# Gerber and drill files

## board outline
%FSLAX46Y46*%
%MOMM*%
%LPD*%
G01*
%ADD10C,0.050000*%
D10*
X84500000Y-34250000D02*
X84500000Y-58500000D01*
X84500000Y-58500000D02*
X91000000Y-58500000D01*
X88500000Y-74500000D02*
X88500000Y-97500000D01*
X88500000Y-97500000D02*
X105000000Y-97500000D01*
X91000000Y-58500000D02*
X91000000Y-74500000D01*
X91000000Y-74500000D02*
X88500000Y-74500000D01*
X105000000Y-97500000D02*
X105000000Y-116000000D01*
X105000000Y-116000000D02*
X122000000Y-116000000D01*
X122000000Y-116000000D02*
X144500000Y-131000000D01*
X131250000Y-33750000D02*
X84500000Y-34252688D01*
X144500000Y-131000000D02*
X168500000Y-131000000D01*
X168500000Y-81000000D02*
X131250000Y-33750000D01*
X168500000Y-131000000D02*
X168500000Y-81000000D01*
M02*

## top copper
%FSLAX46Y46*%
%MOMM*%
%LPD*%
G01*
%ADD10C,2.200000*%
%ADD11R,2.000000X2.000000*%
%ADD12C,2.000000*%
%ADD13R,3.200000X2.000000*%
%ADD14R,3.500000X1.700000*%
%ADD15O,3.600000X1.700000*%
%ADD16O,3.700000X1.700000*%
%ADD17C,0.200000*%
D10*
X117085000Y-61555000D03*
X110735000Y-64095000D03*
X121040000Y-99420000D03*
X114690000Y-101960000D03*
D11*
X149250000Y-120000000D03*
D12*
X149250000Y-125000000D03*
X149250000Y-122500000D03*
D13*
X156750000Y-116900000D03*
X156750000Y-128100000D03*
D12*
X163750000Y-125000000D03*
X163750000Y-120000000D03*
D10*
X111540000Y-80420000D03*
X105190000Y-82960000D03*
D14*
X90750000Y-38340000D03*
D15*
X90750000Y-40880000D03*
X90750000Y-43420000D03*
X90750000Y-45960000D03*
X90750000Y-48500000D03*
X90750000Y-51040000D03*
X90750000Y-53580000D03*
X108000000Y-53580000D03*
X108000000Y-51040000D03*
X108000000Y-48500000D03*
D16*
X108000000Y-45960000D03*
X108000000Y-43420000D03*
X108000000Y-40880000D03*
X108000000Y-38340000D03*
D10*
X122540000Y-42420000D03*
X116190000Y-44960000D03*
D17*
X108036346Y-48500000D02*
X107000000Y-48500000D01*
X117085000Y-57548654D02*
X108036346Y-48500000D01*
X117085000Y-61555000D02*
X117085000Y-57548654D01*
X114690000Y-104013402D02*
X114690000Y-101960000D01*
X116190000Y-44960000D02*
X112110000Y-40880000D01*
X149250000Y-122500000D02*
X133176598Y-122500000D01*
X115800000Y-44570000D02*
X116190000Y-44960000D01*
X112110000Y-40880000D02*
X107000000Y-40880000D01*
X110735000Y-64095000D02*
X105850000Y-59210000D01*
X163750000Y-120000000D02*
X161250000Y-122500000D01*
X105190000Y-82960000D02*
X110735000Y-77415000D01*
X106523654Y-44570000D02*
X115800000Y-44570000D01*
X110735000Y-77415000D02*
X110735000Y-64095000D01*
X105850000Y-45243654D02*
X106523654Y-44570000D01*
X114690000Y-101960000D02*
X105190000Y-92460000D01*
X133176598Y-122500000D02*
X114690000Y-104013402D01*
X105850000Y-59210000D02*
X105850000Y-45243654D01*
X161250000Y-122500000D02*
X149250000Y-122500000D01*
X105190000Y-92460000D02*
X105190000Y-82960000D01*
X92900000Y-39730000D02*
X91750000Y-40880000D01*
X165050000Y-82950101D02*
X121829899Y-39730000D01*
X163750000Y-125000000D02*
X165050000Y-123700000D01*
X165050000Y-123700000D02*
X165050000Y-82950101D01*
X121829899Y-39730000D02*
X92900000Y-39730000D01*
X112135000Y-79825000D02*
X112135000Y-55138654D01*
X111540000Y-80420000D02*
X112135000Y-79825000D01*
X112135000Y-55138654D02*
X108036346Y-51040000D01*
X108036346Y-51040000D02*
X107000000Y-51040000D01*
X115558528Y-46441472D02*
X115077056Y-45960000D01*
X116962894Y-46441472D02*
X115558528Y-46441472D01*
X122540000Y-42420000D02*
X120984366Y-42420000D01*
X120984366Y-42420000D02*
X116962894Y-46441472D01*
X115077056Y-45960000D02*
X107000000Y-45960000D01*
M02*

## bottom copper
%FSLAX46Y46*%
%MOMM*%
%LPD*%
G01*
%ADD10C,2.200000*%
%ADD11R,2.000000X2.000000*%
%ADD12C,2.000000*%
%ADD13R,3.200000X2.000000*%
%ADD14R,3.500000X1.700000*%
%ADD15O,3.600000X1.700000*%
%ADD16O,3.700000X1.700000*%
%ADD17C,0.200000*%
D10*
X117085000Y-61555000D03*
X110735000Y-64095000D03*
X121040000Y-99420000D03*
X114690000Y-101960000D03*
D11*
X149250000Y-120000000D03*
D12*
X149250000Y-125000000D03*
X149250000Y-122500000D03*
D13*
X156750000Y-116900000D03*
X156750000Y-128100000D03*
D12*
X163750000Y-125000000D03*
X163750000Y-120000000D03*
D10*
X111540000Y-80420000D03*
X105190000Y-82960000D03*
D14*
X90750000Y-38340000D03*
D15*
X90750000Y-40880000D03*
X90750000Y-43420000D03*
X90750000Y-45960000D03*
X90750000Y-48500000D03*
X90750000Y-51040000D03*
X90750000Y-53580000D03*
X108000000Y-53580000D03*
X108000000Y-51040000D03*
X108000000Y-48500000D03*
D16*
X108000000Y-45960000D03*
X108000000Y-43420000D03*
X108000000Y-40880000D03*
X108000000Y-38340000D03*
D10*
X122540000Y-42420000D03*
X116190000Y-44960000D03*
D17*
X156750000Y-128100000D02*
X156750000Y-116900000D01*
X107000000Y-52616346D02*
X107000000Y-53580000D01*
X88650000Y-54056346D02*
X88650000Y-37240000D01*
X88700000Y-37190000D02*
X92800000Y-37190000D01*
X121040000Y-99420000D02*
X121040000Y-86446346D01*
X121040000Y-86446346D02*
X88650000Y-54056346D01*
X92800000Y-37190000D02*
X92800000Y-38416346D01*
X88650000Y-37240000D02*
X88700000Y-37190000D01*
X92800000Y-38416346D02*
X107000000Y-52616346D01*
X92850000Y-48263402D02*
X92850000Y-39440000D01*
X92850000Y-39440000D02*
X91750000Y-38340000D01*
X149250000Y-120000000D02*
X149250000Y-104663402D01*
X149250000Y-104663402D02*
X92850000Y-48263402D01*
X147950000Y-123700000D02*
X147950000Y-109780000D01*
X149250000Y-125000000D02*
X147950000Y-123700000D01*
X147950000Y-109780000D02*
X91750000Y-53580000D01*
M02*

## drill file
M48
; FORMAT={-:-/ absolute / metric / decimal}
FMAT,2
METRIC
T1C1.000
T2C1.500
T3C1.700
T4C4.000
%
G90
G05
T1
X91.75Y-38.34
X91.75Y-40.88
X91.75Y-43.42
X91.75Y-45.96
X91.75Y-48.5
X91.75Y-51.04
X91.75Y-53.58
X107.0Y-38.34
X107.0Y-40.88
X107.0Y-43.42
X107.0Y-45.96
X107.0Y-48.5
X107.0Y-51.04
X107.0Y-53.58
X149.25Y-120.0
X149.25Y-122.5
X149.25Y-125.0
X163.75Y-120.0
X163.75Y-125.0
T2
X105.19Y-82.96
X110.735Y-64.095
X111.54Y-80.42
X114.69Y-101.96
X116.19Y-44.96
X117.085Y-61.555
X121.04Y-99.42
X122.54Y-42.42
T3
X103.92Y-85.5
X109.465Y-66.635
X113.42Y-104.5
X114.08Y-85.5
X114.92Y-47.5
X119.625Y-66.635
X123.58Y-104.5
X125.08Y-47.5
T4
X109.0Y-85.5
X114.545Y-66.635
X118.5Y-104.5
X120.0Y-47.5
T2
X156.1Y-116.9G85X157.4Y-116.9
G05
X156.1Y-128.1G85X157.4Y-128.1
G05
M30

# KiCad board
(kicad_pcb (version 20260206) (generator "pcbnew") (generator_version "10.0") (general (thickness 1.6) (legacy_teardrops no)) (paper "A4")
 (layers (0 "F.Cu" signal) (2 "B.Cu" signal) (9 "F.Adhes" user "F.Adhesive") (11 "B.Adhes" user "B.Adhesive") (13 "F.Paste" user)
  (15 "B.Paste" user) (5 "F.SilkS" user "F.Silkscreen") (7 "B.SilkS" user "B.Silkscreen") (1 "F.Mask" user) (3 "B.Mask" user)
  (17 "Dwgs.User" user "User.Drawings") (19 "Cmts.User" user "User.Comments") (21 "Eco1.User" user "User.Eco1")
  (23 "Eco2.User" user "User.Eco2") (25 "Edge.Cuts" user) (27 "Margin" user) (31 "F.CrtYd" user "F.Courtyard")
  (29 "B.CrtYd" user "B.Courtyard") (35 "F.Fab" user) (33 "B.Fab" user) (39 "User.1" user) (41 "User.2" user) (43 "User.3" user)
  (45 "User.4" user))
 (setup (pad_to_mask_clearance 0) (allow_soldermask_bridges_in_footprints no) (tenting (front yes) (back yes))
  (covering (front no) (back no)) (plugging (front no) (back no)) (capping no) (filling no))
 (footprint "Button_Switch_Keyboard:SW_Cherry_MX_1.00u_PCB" (layer "F.Cu") (at 117.085 61.555)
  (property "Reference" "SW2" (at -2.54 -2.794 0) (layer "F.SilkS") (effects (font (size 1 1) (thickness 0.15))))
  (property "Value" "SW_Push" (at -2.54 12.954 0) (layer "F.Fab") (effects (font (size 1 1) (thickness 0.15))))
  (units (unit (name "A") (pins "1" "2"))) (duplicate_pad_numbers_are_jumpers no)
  (pad "" np_thru_hole circle (at -7.62 5.08) (size 1.7 1.7) (drill 1.7) (layers "*.Cu" "*.Mask"))
  (pad "" np_thru_hole circle (at -2.54 5.08) (size 4 4) (drill 4) (layers "*.Cu" "*.Mask"))
  (pad "" np_thru_hole circle (at 2.54 5.08) (size 1.7 1.7) (drill 1.7) (layers "*.Cu" "*.Mask"))
  (pad "1" thru_hole circle (at 0 0) (size 2.2 2.2) (drill 1.5) (layers "*.Cu" "*.Mask") (remove_unused_layers no)
   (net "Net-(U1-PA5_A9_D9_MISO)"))
  (pad "2" thru_hole circle (at -6.35 2.54) (size 2.2 2.2) (drill 1.5) (layers "*.Cu" "*.Mask") (remove_unused_layers no) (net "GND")))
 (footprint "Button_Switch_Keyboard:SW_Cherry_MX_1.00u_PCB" (layer "F.Cu") (at 121.04 99.42)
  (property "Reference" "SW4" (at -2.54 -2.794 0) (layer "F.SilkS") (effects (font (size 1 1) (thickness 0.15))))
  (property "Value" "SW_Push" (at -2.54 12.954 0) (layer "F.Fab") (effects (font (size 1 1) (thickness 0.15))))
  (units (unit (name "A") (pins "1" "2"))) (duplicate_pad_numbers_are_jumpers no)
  (pad "" np_thru_hole circle (at -7.62 5.08) (size 1.7 1.7) (drill 1.7) (layers "*.Cu" "*.Mask"))
  (pad "" np_thru_hole circle (at -2.54 5.08) (size 4 4) (drill 4) (layers "*.Cu" "*.Mask"))
  (pad "" np_thru_hole circle (at 2.54 5.08) (size 1.7 1.7) (drill 1.7) (layers "*.Cu" "*.Mask"))
  (pad "1" thru_hole circle (at 0 0) (size 2.2 2.2) (drill 1.5) (layers "*.Cu" "*.Mask") (remove_unused_layers no)
   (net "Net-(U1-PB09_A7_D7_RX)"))
  (pad "2" thru_hole circle (at -6.35 2.54) (size 2.2 2.2) (drill 1.5) (layers "*.Cu" "*.Mask") (remove_unused_layers no) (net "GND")))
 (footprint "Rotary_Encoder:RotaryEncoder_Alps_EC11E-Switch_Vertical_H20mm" (layer "F.Cu") (at 149.25 120)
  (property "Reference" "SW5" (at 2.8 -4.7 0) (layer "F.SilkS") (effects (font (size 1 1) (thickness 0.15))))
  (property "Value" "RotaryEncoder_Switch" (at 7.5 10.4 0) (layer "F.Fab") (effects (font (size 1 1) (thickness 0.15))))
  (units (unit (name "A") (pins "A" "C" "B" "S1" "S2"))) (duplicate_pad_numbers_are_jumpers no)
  (pad "A" thru_hole rect (at 0 0) (size 2 2) (drill 1) (layers "*.Cu" "*.Mask") (remove_unused_layers no) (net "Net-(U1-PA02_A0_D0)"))
  (pad "B" thru_hole circle (at 0 5) (size 2 2) (drill 1) (layers "*.Cu" "*.Mask") (remove_unused_layers no) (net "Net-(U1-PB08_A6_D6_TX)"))
  (pad "C" thru_hole circle (at 0 2.5) (size 2 2) (drill 1) (layers "*.Cu" "*.Mask") (remove_unused_layers no) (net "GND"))
  (pad "MP" thru_hole rect (at 7.5 -3.1) (size 3.2 2) (drill oval 2.8 1.5) (layers "*.Cu" "*.Mask") (remove_unused_layers no))
  (pad "MP" thru_hole rect (at 7.5 8.1) (size 3.2 2) (drill oval 2.8 1.5) (layers "*.Cu" "*.Mask") (remove_unused_layers no))
  (pad "S1" thru_hole circle (at 14.5 5) (size 2 2) (drill 1) (layers "*.Cu" "*.Mask") (remove_unused_layers no) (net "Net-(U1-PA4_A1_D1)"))
  (pad "S2" thru_hole circle (at 14.5 0) (size 2 2) (drill 1) (layers "*.Cu" "*.Mask") (remove_unused_layers no) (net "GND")))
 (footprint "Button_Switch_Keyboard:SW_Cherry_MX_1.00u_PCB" (layer "F.Cu") (at 111.54 80.42)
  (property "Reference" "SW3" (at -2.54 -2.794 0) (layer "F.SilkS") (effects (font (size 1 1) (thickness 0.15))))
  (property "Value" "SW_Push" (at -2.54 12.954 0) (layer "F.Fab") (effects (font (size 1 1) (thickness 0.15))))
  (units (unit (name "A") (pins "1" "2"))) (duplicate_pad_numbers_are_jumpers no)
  (pad "" np_thru_hole circle (at -7.62 5.08) (size 1.7 1.7) (drill 1.7) (layers "*.Cu" "*.Mask"))
  (pad "" np_thru_hole circle (at -2.54 5.08) (size 4 4) (drill 4) (layers "*.Cu" "*.Mask"))
  (pad "" np_thru_hole circle (at 2.54 5.08) (size 1.7 1.7) (drill 1.7) (layers "*.Cu" "*.Mask"))
  (pad "1" thru_hole circle (at 0 0) (size 2.2 2.2) (drill 1.5) (layers "*.Cu" "*.Mask") (remove_unused_layers no)
   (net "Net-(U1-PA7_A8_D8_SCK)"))
  (pad "2" thru_hole circle (at -6.35 2.54) (size 2.2 2.2) (drill 1.5) (layers "*.Cu" "*.Mask") (remove_unused_layers no) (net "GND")))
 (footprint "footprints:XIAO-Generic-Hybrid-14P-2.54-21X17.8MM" (layer "F.Cu") (at 99.375 45.96)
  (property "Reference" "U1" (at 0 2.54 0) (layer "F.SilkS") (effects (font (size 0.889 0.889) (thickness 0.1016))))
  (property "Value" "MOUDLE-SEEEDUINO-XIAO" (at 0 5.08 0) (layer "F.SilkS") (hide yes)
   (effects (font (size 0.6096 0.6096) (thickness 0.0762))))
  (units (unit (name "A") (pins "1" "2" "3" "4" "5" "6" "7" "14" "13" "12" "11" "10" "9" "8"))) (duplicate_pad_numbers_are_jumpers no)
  (pad "1" thru_hole rect (at -7.625 -7.62) (size 3.5 1.7) (drill 1 (offset -1 0)) (layers "*.Cu" "*.Mask") (remove_unused_layers no)
   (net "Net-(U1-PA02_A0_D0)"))
  (pad "2" thru_hole oval (at -7.625 -5.08) (size 3.6 1.7) (drill 1 (offset -1 0)) (layers "*.Cu" "*.Mask") (remove_unused_layers no)
   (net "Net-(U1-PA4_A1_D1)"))
  (pad "3" thru_hole oval (at -7.625 -2.54) (size 3.6 1.7) (drill 1 (offset -1 0)) (layers "*.Cu" "*.Mask") (remove_unused_layers no)
   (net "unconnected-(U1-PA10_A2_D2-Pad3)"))
  (pad "4" thru_hole oval (at -7.625 0) (size 3.6 1.7) (drill 1 (offset -1 0)) (layers "*.Cu" "*.Mask") (remove_unused_layers no)
   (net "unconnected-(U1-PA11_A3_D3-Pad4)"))
  (pad "5" thru_hole oval (at -7.625 2.54) (size 3.6 1.7) (drill 1 (offset -1 0)) (layers "*.Cu" "*.Mask") (remove_unused_layers no)
   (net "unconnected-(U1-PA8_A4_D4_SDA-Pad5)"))
  (pad "6" thru_hole oval (at -7.625 5.08 180) (size 3.6 1.7) (drill 1 (offset 1 0)) (layers "*.Cu" "*.Mask") (remove_unused_layers no)
   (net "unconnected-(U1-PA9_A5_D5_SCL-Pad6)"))
  (pad "7" thru_hole oval (at -7.625 7.62) (size 3.6 1.7) (drill 1 (offset -1 0)) (layers "*.Cu" "*.Mask") (remove_unused_layers no)
   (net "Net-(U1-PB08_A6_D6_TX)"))
  (pad "8" thru_hole oval (at 7.625 7.62) (size 3.6 1.7) (drill 1 (offset 1 0)) (layers "*.Cu" "*.Mask") (remove_unused_layers no)
   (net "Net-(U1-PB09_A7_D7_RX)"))
  (pad "9" thru_hole oval (at 7.625 5.08) (size 3.6 1.7) (drill 1 (offset 1 0)) (layers "*.Cu" "*.Mask") (remove_unused_layers no)
   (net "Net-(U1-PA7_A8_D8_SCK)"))
  (pad "10" thru_hole oval (at 7.625 2.54) (size 3.6 1.7) (drill 1 (offset 1 0)) (layers "*.Cu" "*.Mask") (remove_unused_layers no)
   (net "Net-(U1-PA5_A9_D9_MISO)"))
  (pad "11" thru_hole oval (at 7.625 0) (size 3.7 1.7) (drill 1 (offset 1 0)) (layers "*.Cu" "*.Mask") (remove_unused_layers no)
   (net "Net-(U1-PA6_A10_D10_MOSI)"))
  (pad "12" thru_hole oval (at 7.625 -2.54) (size 3.7 1.7) (drill 1 (offset 1 0)) (layers "*.Cu" "*.Mask") (remove_unused_layers no)
   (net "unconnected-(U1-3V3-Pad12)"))
  (pad "13" thru_hole oval (at 7.625 -5.08) (size 3.7 1.7) (drill 1 (offset 1 0)) (layers "*.Cu" "*.Mask") (remove_unused_layers no)
   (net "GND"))
  (pad "14" thru_hole oval (at 7.625 -7.62) (size 3.7 1.7) (drill 1 (offset 1 0)) (layers "*.Cu" "*.Mask") (remove_unused_layers no)
   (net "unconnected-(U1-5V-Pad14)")))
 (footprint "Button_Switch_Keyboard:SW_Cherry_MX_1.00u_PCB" (layer "F.Cu") (at 122.54 42.42)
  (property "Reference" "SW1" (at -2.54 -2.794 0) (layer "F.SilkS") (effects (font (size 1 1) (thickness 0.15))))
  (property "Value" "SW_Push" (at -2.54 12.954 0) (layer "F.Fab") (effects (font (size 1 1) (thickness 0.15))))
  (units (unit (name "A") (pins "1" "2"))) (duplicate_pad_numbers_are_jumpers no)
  (pad "" np_thru_hole circle (at -7.62 5.08) (size 1.7 1.7) (drill 1.7) (layers "*.Cu" "*.Mask"))
  (pad "" np_thru_hole circle (at -2.54 5.08) (size 4 4) (drill 4) (layers "*.Cu" "*.Mask"))
  (pad "" np_thru_hole circle (at 2.54 5.08) (size 1.7 1.7) (drill 1.7) (layers "*.Cu" "*.Mask"))
  (pad "1" thru_hole circle (at 0 0) (size 2.2 2.2) (drill 1.5) (layers "*.Cu" "*.Mask") (remove_unused_layers no)
   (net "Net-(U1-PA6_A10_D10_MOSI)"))
  (pad "2" thru_hole circle (at -6.35 2.54) (size 2.2 2.2) (drill 1.5) (layers "*.Cu" "*.Mask") (remove_unused_layers no) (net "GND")))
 (gr_line (start 84.5 34.25) (end 84.5 58.5) (stroke (width 0.05) (type default)) (layer "Edge.Cuts"))
 (gr_line (start 84.5 58.5) (end 91 58.5) (stroke (width 0.05) (type default)) (layer "Edge.Cuts"))
 (gr_line (start 88.5 74.5) (end 88.5 97.5) (stroke (width 0.05) (type default)) (layer "Edge.Cuts"))
 (gr_line (start 88.5 97.5) (end 105 97.5) (stroke (width 0.05) (type default)) (layer "Edge.Cuts"))
 (gr_line (start 91 58.5) (end 91 74.5) (stroke (width 0.05) (type default)) (layer "Edge.Cuts"))
 (gr_line (start 91 74.5) (end 88.5 74.5) (stroke (width 0.05) (type default)) (layer "Edge.Cuts"))
 (gr_line (start 105 97.5) (end 105 116) (stroke (width 0.05) (type default)) (layer "Edge.Cuts"))
 (gr_line (start 105 116) (end 122 116) (stroke (width 0.05) (type default)) (layer "Edge.Cuts"))
 (gr_line (start 122 116) (end 144.5 131) (stroke (width 0.05) (type default)) (layer "Edge.Cuts"))
 (gr_line (start 131.25 33.75) (end 84.5 34.252688) (stroke (width 0.05) (type default)) (layer "Edge.Cuts"))
 (gr_line (start 144.5 131) (end 168.5 131) (stroke (width 0.05) (type default)) (layer "Edge.Cuts"))
 (gr_line (start 168.5 81) (end 131.25 33.75) (stroke (width 0.05) (type default)) (layer "Edge.Cuts"))
 (gr_line (start 168.5 131) (end 168.5 81) (stroke (width 0.05) (type default)) (layer "Edge.Cuts"))
 (segment (start 156.75 128.1) (end 156.75 116.9) (width 0.2) (layer "B.Cu") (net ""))
 (segment (start 108.036346 48.5) (end 107 48.5) (width 0.2) (layer "F.Cu") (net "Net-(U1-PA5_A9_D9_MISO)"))
 (segment (start 117.085 57.548654) (end 108.036346 48.5) (width 0.2) (layer "F.Cu") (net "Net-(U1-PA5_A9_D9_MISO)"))
 (segment (start 117.085 61.555) (end 117.085 57.548654) (width 0.2) (layer "F.Cu") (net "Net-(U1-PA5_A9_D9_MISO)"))
 (segment (start 114.69 104.013402) (end 114.69 101.96) (width 0.2) (layer "F.Cu") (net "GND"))
 (segment (start 116.19 44.96) (end 112.11 40.88) (width 0.2) (layer "F.Cu") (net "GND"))
 (segment (start 149.25 122.5) (end 133.176598 122.5) (width 0.2) (layer "F.Cu") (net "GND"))
 (segment (start 115.8 44.57) (end 116.19 44.96) (width 0.2) (layer "F.Cu") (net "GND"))
 (segment (start 112.11 40.88) (end 107 40.88) (width 0.2) (layer "F.Cu") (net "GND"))
 (segment (start 110.735 64.095) (end 105.85 59.21) (width 0.2) (layer "F.Cu") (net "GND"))
 (segment (start 163.75 120) (end 161.25 122.5) (width 0.2) (layer "F.Cu") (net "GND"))
 (segment (start 105.19 82.96) (end 110.735 77.415) (width 0.2) (layer "F.Cu") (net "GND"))
 (segment (start 106.523654 44.57) (end 115.8 44.57) (width 0.2) (layer "F.Cu") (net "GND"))
 (segment (start 110.735 77.415) (end 110.735 64.095) (width 0.2) (layer "F.Cu") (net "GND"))
 (segment (start 105.85 45.243654) (end 106.523654 44.57) (width 0.2) (layer "F.Cu") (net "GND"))
 (segment (start 114.69 101.96) (end 105.19 92.46) (width 0.2) (layer "F.Cu") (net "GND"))
 (segment (start 133.176598 122.5) (end 114.69 104.013402) (width 0.2) (layer "F.Cu") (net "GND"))
 (segment (start 105.85 59.21) (end 105.85 45.243654) (width 0.2) (layer "F.Cu") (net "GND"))
 (segment (start 161.25 122.5) (end 149.25 122.5) (width 0.2) (layer "F.Cu") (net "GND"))
 (segment (start 105.19 92.46) (end 105.19 82.96) (width 0.2) (layer "F.Cu") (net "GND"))
 (segment (start 107 52.616346) (end 107 53.58) (width 0.2) (layer "B.Cu") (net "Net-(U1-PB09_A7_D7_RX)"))
 (segment (start 88.65 54.056346) (end 88.65 37.24) (width 0.2) (layer "B.Cu") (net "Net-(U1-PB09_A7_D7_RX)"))
 (segment (start 88.7 37.19) (end 92.8 37.19) (width 0.2) (layer "B.Cu") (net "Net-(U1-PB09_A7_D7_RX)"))
 (segment (start 121.04 99.42) (end 121.04 86.446346) (width 0.2) (layer "B.Cu") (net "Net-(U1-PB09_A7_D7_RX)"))
 (segment (start 121.04 86.446346) (end 88.65 54.056346) (width 0.2) (layer "B.Cu") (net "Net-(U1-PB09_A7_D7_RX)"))
 (segment (start 92.8 37.19) (end 92.8 38.416346) (width 0.2) (layer "B.Cu") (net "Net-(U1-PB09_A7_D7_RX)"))
 (segment (start 88.65 37.24) (end 88.7 37.19) (width 0.2) (layer "B.Cu") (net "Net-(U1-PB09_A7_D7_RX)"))
 (segment (start 92.8 38.416346) (end 107 52.616346) (width 0.2) (layer "B.Cu") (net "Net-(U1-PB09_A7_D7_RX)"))
 (segment (start 92.85 48.263402) (end 92.85 39.44) (width 0.2) (layer "B.Cu") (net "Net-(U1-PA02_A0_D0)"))
 (segment (start 92.85 39.44) (end 91.75 38.34) (width 0.2) (layer "B.Cu") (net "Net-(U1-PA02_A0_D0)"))
 (segment (start 149.25 120) (end 149.25 104.663402) (width 0.2) (layer "B.Cu") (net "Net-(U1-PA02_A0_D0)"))
 (segment (start 149.25 104.663402) (end 92.85 48.263402) (width 0.2) (layer "B.Cu") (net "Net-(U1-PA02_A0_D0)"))
 (segment (start 147.95 123.7) (end 147.95 109.78) (width 0.2) (layer "B.Cu") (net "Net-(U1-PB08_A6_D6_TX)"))
 (segment (start 149.25 125) (end 147.95 123.7) (width 0.2) (layer "B.Cu") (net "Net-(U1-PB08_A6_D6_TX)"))
 (segment (start 147.95 109.78) (end 91.75 53.58) (width 0.2) (layer "B.Cu") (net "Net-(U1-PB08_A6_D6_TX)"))
 (segment (start 92.9 39.73) (end 91.75 40.88) (width 0.2) (layer "F.Cu") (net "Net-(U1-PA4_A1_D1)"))
 (segment (start 165.05 82.950101) (end 121.829899 39.73) (width 0.2) (layer "F.Cu") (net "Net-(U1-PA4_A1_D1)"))
 (segment (start 163.75 125) (end 165.05 123.7) (width 0.2) (layer "F.Cu") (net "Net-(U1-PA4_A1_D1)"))
 (segment (start 165.05 123.7) (end 165.05 82.950101) (width 0.2) (layer "F.Cu") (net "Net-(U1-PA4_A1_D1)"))
 (segment (start 121.829899 39.73) (end 92.9 39.73) (width 0.2) (layer "F.Cu") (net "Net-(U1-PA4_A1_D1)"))
 (segment (start 112.135 79.825) (end 112.135 55.138654) (width 0.2) (layer "F.Cu") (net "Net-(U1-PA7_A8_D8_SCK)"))
 (segment (start 111.54 80.42) (end 112.135 79.825) (width 0.2) (layer "F.Cu") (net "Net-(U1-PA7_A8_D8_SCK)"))
 (segment (start 112.135 55.138654) (end 108.036346 51.04) (width 0.2) (layer "F.Cu") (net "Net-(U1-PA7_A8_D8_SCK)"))
 (segment (start 108.036346 51.04) (end 107 51.04) (width 0.2) (layer "F.Cu") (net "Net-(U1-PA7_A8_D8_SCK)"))
 (segment (start 115.558528 46.441472) (end 115.077056 45.96) (width 0.2) (layer "F.Cu") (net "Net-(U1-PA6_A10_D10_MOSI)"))
 (segment (start 116.962894 46.441472) (end 115.558528 46.441472) (width 0.2) (layer "F.Cu") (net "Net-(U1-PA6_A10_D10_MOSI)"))
 (segment (start 122.54 42.42) (end 120.984366 42.42) (width 0.2) (layer "F.Cu") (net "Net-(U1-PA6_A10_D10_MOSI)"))
 (segment (start 120.984366 42.42) (end 116.962894 46.441472) (width 0.2) (layer "F.Cu") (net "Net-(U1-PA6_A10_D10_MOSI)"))
 (segment (start 115.077056 45.96) (end 107 45.96) (width 0.2) (layer "F.Cu") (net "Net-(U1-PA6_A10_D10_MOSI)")))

